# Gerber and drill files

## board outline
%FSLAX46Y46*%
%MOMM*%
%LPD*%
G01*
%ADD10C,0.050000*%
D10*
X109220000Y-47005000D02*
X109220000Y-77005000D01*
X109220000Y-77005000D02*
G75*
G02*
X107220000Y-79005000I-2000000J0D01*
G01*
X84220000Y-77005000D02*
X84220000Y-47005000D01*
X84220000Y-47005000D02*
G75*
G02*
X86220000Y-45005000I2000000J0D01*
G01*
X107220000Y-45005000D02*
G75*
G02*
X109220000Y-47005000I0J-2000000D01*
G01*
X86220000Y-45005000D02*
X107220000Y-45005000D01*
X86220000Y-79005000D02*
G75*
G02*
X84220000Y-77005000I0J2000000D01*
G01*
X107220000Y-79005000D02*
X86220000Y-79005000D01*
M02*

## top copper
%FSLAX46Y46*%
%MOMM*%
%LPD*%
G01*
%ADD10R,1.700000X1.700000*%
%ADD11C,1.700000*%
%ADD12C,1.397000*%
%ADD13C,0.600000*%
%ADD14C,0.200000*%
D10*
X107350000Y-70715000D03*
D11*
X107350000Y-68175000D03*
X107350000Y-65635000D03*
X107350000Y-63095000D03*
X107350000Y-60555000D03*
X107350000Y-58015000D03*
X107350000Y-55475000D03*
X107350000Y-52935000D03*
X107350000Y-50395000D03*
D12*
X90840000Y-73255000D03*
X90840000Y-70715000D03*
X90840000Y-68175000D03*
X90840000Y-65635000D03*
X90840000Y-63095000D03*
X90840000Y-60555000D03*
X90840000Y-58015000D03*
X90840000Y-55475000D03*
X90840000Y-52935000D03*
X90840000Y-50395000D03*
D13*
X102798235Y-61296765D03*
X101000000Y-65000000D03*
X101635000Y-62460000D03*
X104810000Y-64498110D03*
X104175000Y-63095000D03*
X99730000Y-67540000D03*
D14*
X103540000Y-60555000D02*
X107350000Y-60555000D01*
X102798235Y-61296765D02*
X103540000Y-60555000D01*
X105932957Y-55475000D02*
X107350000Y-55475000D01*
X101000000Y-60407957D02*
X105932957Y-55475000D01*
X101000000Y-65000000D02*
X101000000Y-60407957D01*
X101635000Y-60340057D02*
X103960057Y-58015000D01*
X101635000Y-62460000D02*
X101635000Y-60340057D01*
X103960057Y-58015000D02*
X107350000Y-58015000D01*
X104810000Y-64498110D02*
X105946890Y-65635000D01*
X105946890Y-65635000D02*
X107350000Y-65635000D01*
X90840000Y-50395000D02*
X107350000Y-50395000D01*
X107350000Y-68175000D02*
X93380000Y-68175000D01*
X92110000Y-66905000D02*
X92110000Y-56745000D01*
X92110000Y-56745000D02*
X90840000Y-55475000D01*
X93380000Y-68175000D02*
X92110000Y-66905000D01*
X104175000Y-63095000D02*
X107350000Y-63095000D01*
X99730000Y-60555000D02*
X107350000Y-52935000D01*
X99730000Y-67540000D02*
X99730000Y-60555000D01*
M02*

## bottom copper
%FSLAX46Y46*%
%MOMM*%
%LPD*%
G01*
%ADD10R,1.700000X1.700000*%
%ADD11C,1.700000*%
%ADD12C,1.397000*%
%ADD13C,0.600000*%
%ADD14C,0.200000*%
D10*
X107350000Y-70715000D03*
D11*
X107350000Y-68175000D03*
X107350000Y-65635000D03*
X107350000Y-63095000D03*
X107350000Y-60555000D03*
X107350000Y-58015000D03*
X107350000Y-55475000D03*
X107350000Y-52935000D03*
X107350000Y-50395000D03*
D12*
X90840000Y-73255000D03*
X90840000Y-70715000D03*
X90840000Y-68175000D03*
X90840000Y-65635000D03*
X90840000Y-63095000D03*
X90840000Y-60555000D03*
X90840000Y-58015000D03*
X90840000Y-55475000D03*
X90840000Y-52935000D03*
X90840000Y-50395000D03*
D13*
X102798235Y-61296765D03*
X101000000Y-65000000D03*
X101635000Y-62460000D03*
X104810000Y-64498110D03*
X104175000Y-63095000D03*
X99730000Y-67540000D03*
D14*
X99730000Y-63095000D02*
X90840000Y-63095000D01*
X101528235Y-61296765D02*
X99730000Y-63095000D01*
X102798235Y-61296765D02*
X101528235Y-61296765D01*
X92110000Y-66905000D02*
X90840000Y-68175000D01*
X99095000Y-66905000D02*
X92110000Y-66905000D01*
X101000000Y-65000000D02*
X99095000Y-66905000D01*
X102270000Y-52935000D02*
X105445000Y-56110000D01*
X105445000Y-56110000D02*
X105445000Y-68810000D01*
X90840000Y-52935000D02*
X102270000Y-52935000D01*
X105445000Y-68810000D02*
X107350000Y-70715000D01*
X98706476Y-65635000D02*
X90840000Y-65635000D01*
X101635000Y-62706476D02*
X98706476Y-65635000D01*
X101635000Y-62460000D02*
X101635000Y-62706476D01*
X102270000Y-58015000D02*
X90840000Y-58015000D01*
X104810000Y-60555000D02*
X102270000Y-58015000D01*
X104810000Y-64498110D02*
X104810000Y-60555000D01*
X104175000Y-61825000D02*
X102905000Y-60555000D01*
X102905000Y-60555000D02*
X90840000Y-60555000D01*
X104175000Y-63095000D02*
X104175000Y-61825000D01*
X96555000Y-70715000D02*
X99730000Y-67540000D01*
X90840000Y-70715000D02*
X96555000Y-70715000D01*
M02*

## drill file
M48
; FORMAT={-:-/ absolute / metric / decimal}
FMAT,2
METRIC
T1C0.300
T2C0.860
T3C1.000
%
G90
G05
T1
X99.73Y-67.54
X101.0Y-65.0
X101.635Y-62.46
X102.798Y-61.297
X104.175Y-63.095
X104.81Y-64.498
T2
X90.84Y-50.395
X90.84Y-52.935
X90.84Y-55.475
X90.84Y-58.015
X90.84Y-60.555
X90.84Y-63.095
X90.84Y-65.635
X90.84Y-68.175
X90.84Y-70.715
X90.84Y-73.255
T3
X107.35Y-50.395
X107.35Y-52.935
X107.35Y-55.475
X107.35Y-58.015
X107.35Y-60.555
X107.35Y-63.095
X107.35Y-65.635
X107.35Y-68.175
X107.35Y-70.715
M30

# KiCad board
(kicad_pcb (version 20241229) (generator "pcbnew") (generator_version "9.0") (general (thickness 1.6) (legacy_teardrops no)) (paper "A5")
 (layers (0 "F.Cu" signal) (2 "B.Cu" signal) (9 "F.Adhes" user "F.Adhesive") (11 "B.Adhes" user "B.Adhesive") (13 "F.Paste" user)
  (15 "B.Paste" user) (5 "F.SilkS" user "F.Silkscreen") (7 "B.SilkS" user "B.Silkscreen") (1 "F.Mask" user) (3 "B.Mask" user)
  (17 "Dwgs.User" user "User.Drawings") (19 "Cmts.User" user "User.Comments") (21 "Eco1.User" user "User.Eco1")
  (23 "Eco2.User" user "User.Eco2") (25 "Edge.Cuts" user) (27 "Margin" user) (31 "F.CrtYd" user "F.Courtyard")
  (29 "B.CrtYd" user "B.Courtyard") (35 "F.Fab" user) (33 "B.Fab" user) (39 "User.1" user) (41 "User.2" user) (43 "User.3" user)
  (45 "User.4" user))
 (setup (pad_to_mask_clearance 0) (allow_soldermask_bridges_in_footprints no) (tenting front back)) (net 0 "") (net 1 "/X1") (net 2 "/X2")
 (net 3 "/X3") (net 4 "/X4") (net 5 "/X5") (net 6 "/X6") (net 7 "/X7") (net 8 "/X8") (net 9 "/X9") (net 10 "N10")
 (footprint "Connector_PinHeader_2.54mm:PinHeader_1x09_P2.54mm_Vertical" (layer "F.Cu") (at 107.35 50.395)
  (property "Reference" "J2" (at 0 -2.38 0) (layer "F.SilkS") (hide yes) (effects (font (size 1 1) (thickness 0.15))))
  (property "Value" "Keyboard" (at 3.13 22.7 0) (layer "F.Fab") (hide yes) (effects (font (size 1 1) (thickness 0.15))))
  (pad "1" thru_hole rect (at 0 20.32) (size 1.7 1.7) (drill 1) (layers "*.Cu" "*.Mask") (remove_unused_layers no) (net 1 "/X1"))
  (pad "2" thru_hole circle (at 0 17.78) (size 1.7 1.7) (drill 1) (layers "*.Cu" "*.Mask") (remove_unused_layers no) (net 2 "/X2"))
  (pad "3" thru_hole circle (at 0 15.24) (size 1.7 1.7) (drill 1) (layers "*.Cu" "*.Mask") (remove_unused_layers no) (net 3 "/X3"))
  (pad "4" thru_hole circle (at 0 12.7) (size 1.7 1.7) (drill 1) (layers "*.Cu" "*.Mask") (remove_unused_layers no) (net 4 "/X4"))
  (pad "5" thru_hole circle (at 0 10.16) (size 1.7 1.7) (drill 1) (layers "*.Cu" "*.Mask") (remove_unused_layers no) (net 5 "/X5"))
  (pad "6" thru_hole circle (at 0 7.62) (size 1.7 1.7) (drill 1) (layers "*.Cu" "*.Mask") (remove_unused_layers no) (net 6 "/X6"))
  (pad "7" thru_hole circle (at 0 5.08) (size 1.7 1.7) (drill 1) (layers "*.Cu" "*.Mask") (remove_unused_layers no) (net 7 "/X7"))
  (pad "8" thru_hole circle (at 0 2.54) (size 1.7 1.7) (drill 1) (layers "*.Cu" "*.Mask") (remove_unused_layers no) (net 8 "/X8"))
  (pad "9" thru_hole circle (at 0 0) (size 1.7 1.7) (drill 1) (layers "*.Cu" "*.Mask") (remove_unused_layers no) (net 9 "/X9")))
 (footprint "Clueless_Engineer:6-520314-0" (layer "F.Cu") (at 90.84 61.825 -90)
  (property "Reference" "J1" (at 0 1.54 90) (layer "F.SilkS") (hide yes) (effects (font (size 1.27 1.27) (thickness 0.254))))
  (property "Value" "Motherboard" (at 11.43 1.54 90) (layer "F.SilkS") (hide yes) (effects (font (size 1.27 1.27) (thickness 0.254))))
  (pad "1" thru_hole circle (at 11.43 0 270) (size 1.397 1.397) (drill 0.86) (layers "*.Cu" "*.Mask") (remove_unused_layers no)
   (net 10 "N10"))
  (pad "2" thru_hole circle (at 8.89 0 270) (size 1.397 1.397) (drill 0.86) (layers "*.Cu" "*.Mask") (remove_unused_layers no) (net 8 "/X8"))
  (pad "3" thru_hole circle (at 6.35 0 270) (size 1.397 1.397) (drill 0.86) (layers "*.Cu" "*.Mask") (remove_unused_layers no) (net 7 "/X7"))
  (pad "4" thru_hole circle (at 3.81 0 270) (size 1.397 1.397) (drill 0.86) (layers "*.Cu" "*.Mask") (remove_unused_layers no) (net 6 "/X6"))
  (pad "5" thru_hole circle (at 1.27 0 270) (size 1.397 1.397) (drill 0.86) (layers "*.Cu" "*.Mask") (remove_unused_layers no) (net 5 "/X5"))
  (pad "6" thru_hole circle (at -1.27 0 270) (size 1.397 1.397) (drill 0.86) (layers "*.Cu" "*.Mask") (remove_unused_layers no)
   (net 4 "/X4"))
  (pad "7" thru_hole circle (at -3.81 0 270) (size 1.397 1.397) (drill 0.86) (layers "*.Cu" "*.Mask") (remove_unused_layers no)
   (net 3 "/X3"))
  (pad "8" thru_hole circle (at -6.35 0 270) (size 1.397 1.397) (drill 0.86) (layers "*.Cu" "*.Mask") (remove_unused_layers no)
   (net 2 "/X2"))
  (pad "9" thru_hole circle (at -8.89 0 270) (size 1.397 1.397) (drill 0.86) (layers "*.Cu" "*.Mask") (remove_unused_layers no)
   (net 1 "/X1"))
  (pad "10" thru_hole circle (at -11.43 0 270) (size 1.397 1.397) (drill 0.86) (layers "*.Cu" "*.Mask") (remove_unused_layers no)
   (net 9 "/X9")))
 (gr_line (start 109.22 47.005) (end 109.22 77.005) (stroke (width 0.05) (type default)) (layer "Edge.Cuts"))
 (gr_arc (start 109.22 77.005) (mid 108.634214 78.419214) (end 107.22 79.005) (stroke (width 0.05) (type default)) (layer "Edge.Cuts"))
 (gr_line (start 84.22 77.005) (end 84.22 47.005) (stroke (width 0.05) (type default)) (layer "Edge.Cuts"))
 (gr_arc (start 84.22 47.005) (mid 84.805786 45.590786) (end 86.22 45.005) (stroke (width 0.05) (type default)) (layer "Edge.Cuts"))
 (gr_arc (start 107.22 45.005) (mid 108.634214 45.590786) (end 109.22 47.005) (stroke (width 0.05) (type default)) (layer "Edge.Cuts"))
 (gr_line (start 86.22 45.005) (end 107.22 45.005) (stroke (width 0.05) (type default)) (layer "Edge.Cuts"))
 (gr_arc (start 86.22 79.005) (mid 84.805786 78.419214) (end 84.22 77.005) (stroke (width 0.05) (type default)) (layer "Edge.Cuts"))
 (gr_line (start 107.22 79.005) (end 86.22 79.005) (stroke (width 0.05) (type default)) (layer "Edge.Cuts"))
 (segment (start 103.54 60.555) (end 107.35 60.555) (width 0.2) (layer "F.Cu") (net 5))
 (segment (start 102.798235 61.296765) (end 103.54 60.555) (width 0.2) (layer "F.Cu") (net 5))
 (via (at 102.798235 61.296765) (size 0.6) (drill 0.3) (layers "F.Cu" "B.Cu") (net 5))
 (segment (start 99.73 63.095) (end 90.84 63.095) (width 0.2) (layer "B.Cu") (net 5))
 (segment (start 101.528235 61.296765) (end 99.73 63.095) (width 0.2) (layer "B.Cu") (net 5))
 (segment (start 102.798235 61.296765) (end 101.528235 61.296765) (width 0.2) (layer "B.Cu") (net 5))
 (segment (start 105.932957 55.475) (end 107.35 55.475) (width 0.2) (layer "F.Cu") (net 7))
 (segment (start 101 60.407957) (end 105.932957 55.475) (width 0.2) (layer "F.Cu") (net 7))
 (segment (start 101 65) (end 101 60.407957) (width 0.2) (layer "F.Cu") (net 7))
 (via (at 101 65) (size 0.6) (drill 0.3) (layers "F.Cu" "B.Cu") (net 7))
 (segment (start 92.11 66.905) (end 90.84 68.175) (width 0.2) (layer "B.Cu") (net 7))
 (segment (start 99.095 66.905) (end 92.11 66.905) (width 0.2) (layer "B.Cu") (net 7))
 (segment (start 101 65) (end 99.095 66.905) (width 0.2) (layer "B.Cu") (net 7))
 (segment (start 102.27 52.935) (end 105.445 56.11) (width 0.2) (layer "B.Cu") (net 1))
 (segment (start 105.445 56.11) (end 105.445 68.81) (width 0.2) (layer "B.Cu") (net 1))
 (segment (start 90.84 52.935) (end 102.27 52.935) (width 0.2) (layer "B.Cu") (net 1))
 (segment (start 105.445 68.81) (end 107.35 70.715) (width 0.2) (layer "B.Cu") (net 1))
 (segment (start 101.635 60.340057) (end 103.960057 58.015) (width 0.2) (layer "F.Cu") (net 6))
 (segment (start 101.635 62.46) (end 101.635 60.340057) (width 0.2) (layer "F.Cu") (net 6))
 (segment (start 103.960057 58.015) (end 107.35 58.015) (width 0.2) (layer "F.Cu") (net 6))
 (via (at 101.635 62.46) (size 0.6) (drill 0.3) (layers "F.Cu" "B.Cu") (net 6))
 (segment (start 98.706476 65.635) (end 90.84 65.635) (width 0.2) (layer "B.Cu") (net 6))
 (segment (start 101.635 62.706476) (end 98.706476 65.635) (width 0.2) (layer "B.Cu") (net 6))
 (segment (start 101.635 62.46) (end 101.635 62.706476) (width 0.2) (layer "B.Cu") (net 6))
 (segment (start 104.81 64.49811) (end 105.94689 65.635) (width 0.2) (layer "F.Cu") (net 3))
 (segment (start 105.94689 65.635) (end 107.35 65.635) (width 0.2) (layer "F.Cu") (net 3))
 (via (at 104.81 64.49811) (size 0.6) (drill 0.3) (layers "F.Cu" "B.Cu") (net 3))
 (segment (start 102.27 58.015) (end 90.84 58.015) (width 0.2) (layer "B.Cu") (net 3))
 (segment (start 104.81 60.555) (end 102.27 58.015) (width 0.2) (layer "B.Cu") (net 3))
 (segment (start 104.81 64.49811) (end 104.81 60.555) (width 0.2) (layer "B.Cu") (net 3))
 (segment (start 90.84 50.395) (end 107.35 50.395) (width 0.2) (layer "F.Cu") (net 9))
 (segment (start 107.35 68.175) (end 93.38 68.175) (width 0.2) (layer "F.Cu") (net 2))
 (segment (start 92.11 66.905) (end 92.11 56.745) (width 0.2) (layer "F.Cu") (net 2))
 (segment (start 92.11 56.745) (end 90.84 55.475) (width 0.2) (layer "F.Cu") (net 2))
 (segment (start 93.38 68.175) (end 92.11 66.905) (width 0.2) (layer "F.Cu") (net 2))
 (segment (start 104.175 63.095) (end 107.35 63.095) (width 0.2) (layer "F.Cu") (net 4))
 (via (at 104.175 63.095) (size 0.6) (drill 0.3) (layers "F.Cu" "B.Cu") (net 4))
 (segment (start 104.175 61.825) (end 102.905 60.555) (width 0.2) (layer "B.Cu") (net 4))
 (segment (start 102.905 60.555) (end 90.84 60.555) (width 0.2) (layer "B.Cu") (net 4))
 (segment (start 104.175 63.095) (end 104.175 61.825) (width 0.2) (layer "B.Cu") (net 4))
 (segment (start 99.73 60.555) (end 107.35 52.935) (width 0.2) (layer "F.Cu") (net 8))
 (segment (start 99.73 67.54) (end 99.73 60.555) (width 0.2) (layer "F.Cu") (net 8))
 (via (at 99.73 67.54) (size 0.6) (drill 0.3) (layers "F.Cu" "B.Cu") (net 8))
 (segment (start 96.555 70.715) (end 99.73 67.54) (width 0.2) (layer "B.Cu") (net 8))
 (segment (start 90.84 70.715) (end 96.555 70.715) (width 0.2) (layer "B.Cu") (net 8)))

